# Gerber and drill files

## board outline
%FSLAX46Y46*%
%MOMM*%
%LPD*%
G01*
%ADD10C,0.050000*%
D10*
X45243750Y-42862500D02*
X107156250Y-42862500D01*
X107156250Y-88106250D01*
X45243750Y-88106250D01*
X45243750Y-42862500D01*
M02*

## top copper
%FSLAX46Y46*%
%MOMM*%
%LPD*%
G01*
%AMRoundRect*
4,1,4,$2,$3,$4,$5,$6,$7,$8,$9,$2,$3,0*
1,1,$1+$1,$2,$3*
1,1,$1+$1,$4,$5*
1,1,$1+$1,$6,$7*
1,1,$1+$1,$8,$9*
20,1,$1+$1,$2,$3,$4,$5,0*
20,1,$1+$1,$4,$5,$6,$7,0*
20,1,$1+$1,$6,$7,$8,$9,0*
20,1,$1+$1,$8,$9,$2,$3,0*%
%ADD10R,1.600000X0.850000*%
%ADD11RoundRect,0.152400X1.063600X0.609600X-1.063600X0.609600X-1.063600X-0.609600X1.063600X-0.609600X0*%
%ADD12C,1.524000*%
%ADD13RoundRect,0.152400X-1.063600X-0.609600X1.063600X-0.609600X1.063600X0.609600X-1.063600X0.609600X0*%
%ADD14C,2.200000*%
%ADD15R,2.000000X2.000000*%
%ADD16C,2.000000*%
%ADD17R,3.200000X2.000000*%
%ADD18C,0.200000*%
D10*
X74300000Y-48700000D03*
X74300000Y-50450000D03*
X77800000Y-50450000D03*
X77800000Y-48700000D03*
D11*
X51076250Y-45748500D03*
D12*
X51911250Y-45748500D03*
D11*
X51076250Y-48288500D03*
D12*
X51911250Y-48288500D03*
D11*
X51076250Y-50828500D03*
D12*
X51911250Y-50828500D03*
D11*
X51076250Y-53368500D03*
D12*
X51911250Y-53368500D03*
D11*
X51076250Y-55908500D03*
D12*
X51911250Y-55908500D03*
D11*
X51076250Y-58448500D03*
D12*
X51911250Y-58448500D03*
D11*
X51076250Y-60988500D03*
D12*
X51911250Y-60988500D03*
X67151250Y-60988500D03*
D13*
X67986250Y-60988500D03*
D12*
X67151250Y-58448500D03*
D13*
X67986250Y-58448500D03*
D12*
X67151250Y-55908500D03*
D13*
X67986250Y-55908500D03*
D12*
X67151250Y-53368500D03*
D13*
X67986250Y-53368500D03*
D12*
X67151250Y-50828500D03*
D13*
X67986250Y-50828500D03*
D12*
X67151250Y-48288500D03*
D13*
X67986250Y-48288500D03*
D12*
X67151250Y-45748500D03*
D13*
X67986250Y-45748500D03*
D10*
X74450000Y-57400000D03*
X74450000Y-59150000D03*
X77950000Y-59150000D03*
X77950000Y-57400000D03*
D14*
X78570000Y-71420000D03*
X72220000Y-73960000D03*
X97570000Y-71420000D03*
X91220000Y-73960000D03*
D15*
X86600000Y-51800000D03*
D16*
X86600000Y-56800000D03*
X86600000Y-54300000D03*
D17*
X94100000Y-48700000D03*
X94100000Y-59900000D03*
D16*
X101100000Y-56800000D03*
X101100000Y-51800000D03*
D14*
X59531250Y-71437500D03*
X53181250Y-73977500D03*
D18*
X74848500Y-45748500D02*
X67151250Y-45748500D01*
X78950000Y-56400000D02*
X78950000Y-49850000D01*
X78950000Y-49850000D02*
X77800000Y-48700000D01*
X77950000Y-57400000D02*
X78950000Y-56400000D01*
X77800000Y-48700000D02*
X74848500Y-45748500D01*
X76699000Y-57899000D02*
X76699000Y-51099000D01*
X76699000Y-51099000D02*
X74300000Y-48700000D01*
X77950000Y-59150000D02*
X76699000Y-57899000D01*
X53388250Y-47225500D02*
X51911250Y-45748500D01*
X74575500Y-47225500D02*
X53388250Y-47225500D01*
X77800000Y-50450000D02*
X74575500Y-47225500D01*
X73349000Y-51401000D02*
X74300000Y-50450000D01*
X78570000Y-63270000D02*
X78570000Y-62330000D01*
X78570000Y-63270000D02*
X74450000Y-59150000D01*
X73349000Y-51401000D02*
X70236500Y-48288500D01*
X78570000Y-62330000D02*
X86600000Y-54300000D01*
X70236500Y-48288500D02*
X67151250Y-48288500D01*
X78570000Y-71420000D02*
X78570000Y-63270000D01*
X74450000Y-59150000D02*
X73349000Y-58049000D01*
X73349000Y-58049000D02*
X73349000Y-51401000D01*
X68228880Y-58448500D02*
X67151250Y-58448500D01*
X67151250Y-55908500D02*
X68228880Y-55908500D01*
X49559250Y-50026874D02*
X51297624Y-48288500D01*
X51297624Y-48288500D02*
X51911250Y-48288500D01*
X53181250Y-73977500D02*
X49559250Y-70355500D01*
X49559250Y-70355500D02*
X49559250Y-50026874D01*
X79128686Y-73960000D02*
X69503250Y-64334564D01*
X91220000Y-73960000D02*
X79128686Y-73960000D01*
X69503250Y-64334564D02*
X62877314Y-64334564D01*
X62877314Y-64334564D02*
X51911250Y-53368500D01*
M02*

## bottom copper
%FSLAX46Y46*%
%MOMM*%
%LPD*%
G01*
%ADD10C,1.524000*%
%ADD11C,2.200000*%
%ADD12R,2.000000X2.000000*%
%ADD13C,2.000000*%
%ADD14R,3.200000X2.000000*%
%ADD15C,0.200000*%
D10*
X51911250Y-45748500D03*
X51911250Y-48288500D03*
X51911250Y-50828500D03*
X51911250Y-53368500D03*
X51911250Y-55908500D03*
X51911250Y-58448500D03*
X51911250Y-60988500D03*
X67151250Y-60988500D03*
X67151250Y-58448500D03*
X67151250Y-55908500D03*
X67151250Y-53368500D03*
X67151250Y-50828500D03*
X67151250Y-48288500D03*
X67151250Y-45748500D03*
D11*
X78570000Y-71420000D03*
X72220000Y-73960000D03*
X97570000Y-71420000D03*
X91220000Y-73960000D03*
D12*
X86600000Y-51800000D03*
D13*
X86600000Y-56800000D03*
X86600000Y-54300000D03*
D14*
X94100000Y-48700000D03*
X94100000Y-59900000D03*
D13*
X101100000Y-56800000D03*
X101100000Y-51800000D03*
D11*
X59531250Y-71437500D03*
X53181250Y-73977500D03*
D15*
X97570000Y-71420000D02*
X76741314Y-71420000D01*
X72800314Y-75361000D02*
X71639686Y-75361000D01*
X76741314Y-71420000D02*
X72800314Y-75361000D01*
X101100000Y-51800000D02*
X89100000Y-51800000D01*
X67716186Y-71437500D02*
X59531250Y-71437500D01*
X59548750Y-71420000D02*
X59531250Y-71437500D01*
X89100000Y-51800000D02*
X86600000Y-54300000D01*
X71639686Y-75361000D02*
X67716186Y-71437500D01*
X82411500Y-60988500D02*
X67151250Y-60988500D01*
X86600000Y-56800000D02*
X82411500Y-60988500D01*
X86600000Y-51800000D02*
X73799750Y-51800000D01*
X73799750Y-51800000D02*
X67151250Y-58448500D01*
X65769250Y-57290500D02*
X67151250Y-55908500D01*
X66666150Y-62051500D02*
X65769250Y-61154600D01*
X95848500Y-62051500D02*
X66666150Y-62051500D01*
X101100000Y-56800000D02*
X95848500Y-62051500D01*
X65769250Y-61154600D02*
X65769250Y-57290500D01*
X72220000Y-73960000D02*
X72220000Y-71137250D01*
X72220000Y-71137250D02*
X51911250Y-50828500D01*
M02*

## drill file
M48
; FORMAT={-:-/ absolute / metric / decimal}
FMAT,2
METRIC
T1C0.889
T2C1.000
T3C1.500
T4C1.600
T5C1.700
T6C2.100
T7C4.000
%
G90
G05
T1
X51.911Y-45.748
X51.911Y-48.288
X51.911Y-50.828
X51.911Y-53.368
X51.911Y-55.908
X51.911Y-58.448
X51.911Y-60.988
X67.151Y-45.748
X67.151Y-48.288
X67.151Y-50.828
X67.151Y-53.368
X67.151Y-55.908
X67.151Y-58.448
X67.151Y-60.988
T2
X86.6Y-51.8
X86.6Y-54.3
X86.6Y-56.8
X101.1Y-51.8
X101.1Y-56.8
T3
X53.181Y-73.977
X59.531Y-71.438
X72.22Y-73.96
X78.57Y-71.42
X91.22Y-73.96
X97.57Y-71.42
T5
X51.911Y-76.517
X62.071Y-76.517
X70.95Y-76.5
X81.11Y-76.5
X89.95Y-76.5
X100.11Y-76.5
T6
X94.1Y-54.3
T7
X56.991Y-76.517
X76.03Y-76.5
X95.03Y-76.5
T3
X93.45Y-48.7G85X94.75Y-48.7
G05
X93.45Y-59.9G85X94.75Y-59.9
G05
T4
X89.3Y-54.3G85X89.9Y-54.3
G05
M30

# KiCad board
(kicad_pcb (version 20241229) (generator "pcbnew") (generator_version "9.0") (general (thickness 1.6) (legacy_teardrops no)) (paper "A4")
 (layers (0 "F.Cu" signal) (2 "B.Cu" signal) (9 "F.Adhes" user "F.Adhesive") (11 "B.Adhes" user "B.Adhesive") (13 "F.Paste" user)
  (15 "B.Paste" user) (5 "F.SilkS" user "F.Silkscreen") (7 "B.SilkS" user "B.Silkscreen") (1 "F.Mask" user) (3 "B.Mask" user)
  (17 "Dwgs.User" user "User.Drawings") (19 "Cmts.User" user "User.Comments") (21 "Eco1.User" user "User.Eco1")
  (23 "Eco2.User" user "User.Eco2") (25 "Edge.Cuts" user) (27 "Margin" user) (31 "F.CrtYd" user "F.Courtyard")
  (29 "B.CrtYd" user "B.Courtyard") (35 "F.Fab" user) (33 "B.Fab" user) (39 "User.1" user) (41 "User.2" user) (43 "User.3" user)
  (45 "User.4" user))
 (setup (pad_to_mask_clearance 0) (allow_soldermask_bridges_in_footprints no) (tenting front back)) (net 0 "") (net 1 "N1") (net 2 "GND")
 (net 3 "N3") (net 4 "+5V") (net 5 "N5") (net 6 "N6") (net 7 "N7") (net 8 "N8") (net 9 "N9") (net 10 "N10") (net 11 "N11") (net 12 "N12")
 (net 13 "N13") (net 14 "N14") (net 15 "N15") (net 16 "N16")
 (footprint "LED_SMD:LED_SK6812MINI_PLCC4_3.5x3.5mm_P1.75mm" (layer "F.Cu") (at 76.05 49.575)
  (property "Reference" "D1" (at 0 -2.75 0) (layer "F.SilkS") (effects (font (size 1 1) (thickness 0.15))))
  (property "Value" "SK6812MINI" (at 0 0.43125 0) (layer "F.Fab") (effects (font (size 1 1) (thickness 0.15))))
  (pad "1" smd rect (at -1.75 -0.875) (size 1.6 0.85) (layers "F.Cu" "F.Mask" "F.Paste") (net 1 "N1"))
  (pad "2" smd rect (at -1.75 0.875) (size 1.6 0.85) (layers "F.Cu" "F.Mask" "F.Paste") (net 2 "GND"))
  (pad "3" smd rect (at 1.75 0.875) (size 1.6 0.85) (layers "F.Cu" "F.Mask" "F.Paste") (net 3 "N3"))
  (pad "4" smd rect (at 1.75 -0.875) (size 1.6 0.85) (layers "F.Cu" "F.Mask" "F.Paste") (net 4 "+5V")))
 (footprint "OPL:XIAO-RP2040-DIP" (layer "F.Cu") (at 59.53125 53.3685)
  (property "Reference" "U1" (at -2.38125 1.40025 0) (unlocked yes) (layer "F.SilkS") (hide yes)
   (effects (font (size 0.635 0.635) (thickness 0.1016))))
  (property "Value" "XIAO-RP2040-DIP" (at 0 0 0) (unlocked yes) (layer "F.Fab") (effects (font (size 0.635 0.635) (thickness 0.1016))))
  (pad "1" smd roundrect (at -8.455 -7.62 180) (size 2.432 1.524) (layers "F.Cu" "F.Mask") (roundrect_rratio 0.1) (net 3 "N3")
   (thermal_bridge_angle 45))
  (pad "1" thru_hole circle (at -7.62 -7.62 180) (size 1.524 1.524) (drill 0.889) (layers "*.Cu" "*.Mask") (remove_unused_layers no)
   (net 3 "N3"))
  (pad "2" smd roundrect (at -8.455 -5.08 180) (size 2.432 1.524) (layers "F.Cu" "F.Mask") (roundrect_rratio 0.1) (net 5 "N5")
   (thermal_bridge_angle 45))
  (pad "2" thru_hole circle (at -7.62 -5.08 180) (size 1.524 1.524) (drill 0.889) (layers "*.Cu" "*.Mask") (remove_unused_layers no)
   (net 5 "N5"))
  (pad "3" smd roundrect (at -8.455 -2.54 180) (size 2.432 1.524) (layers "F.Cu" "F.Mask") (roundrect_rratio 0.1) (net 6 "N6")
   (thermal_bridge_angle 45))
  (pad "3" thru_hole circle (at -7.62 -2.54 180) (size 1.524 1.524) (drill 0.889) (layers "*.Cu" "*.Mask") (remove_unused_layers no)
   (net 6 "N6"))
  (pad "4" smd roundrect (at -8.455 0 180) (size 2.432 1.524) (layers "F.Cu" "F.Mask") (roundrect_rratio 0.1) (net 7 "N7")
   (thermal_bridge_angle 45))
  (pad "4" thru_hole circle (at -7.62 0 180) (size 1.524 1.524) (drill 0.889) (layers "*.Cu" "*.Mask") (remove_unused_layers no)
   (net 7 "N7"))
  (pad "5" smd roundrect (at -8.455 2.54 180) (size 2.432 1.524) (layers "F.Cu" "F.Mask") (roundrect_rratio 0.1) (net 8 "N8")
   (thermal_bridge_angle 45))
  (pad "5" thru_hole circle (at -7.62 2.54 180) (size 1.524 1.524) (drill 0.889) (layers "*.Cu" "*.Mask") (remove_unused_layers no)
   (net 8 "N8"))
  (pad "6" smd roundrect (at -8.455 5.08 180) (size 2.432 1.524) (layers "F.Cu" "F.Mask") (roundrect_rratio 0.1) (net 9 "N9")
   (thermal_bridge_angle 45))
  (pad "6" thru_hole circle (at -7.62 5.08 180) (size 1.524 1.524) (drill 0.889) (layers "*.Cu" "*.Mask") (remove_unused_layers no)
   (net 9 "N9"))
  (pad "7" smd roundrect (at -8.455 7.62 180) (size 2.432 1.524) (layers "F.Cu" "F.Mask") (roundrect_rratio 0.1) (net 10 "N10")
   (thermal_bridge_angle 45))
  (pad "7" thru_hole circle (at -7.62 7.62 180) (size 1.524 1.524) (drill 0.889) (layers "*.Cu" "*.Mask") (remove_unused_layers no)
   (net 10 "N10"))
  (pad "8" thru_hole circle (at 7.62 7.62) (size 1.524 1.524) (drill 0.889) (layers "*.Cu" "*.Mask") (remove_unused_layers no)
   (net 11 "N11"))
  (pad "8" smd roundrect (at 8.455 7.62) (size 2.432 1.524) (layers "F.Cu" "F.Mask") (roundrect_rratio 0.1) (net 11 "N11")
   (thermal_bridge_angle 45))
  (pad "9" thru_hole circle (at 7.62 5.08) (size 1.524 1.524) (drill 0.889) (layers "*.Cu" "*.Mask") (remove_unused_layers no)
   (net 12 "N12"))
  (pad "9" smd roundrect (at 8.455 5.08) (size 2.432 1.524) (layers "F.Cu" "F.Mask") (roundrect_rratio 0.1) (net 12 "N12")
   (thermal_bridge_angle 45))
  (pad "10" thru_hole circle (at 7.62 2.54) (size 1.524 1.524) (drill 0.889) (layers "*.Cu" "*.Mask") (remove_unused_layers no)
   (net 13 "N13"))
  (pad "10" smd roundrect (at 8.455 2.54) (size 2.432 1.524) (layers "F.Cu" "F.Mask") (roundrect_rratio 0.1) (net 13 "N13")
   (thermal_bridge_angle 45))
  (pad "11" thru_hole circle (at 7.62 0) (size 1.524 1.524) (drill 0.889) (layers "*.Cu" "*.Mask") (remove_unused_layers no) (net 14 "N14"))
  (pad "11" smd roundrect (at 8.455 0) (size 2.432 1.524) (layers "F.Cu" "F.Mask") (roundrect_rratio 0.1) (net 14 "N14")
   (thermal_bridge_angle 45))
  (pad "12" thru_hole circle (at 7.62 -2.54) (size 1.524 1.524) (drill 0.889) (layers "*.Cu" "*.Mask") (remove_unused_layers no)
   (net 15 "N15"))
  (pad "12" smd roundrect (at 8.455 -2.54) (size 2.432 1.524) (layers "F.Cu" "F.Mask") (roundrect_rratio 0.1) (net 15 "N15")
   (thermal_bridge_angle 45))
  (pad "13" thru_hole circle (at 7.62 -5.08) (size 1.524 1.524) (drill 0.889) (layers "*.Cu" "*.Mask") (remove_unused_layers no)
   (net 2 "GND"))
  (pad "13" smd roundrect (at 8.455 -5.08) (size 2.432 1.524) (layers "F.Cu" "F.Mask") (roundrect_rratio 0.1) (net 2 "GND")
   (thermal_bridge_angle 45))
  (pad "14" thru_hole circle (at 7.62 -7.62) (size 1.524 1.524) (drill 0.889) (layers "*.Cu" "*.Mask") (remove_unused_layers no)
   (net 4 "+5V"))
  (pad "14" smd roundrect (at 8.455 -7.62) (size 2.432 1.524) (layers "F.Cu" "F.Mask") (roundrect_rratio 0.1) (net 4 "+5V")
   (thermal_bridge_angle 45)))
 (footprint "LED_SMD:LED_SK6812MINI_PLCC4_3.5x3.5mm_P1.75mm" (layer "F.Cu") (at 76.2 58.275)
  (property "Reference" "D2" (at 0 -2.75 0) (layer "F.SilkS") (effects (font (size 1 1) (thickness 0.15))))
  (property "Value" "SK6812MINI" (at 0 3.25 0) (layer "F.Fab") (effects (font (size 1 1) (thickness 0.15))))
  (pad "1" smd rect (at -1.75 -0.875) (size 1.6 0.85) (layers "F.Cu" "F.Mask" "F.Paste") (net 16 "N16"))
  (pad "2" smd rect (at -1.75 0.875) (size 1.6 0.85) (layers "F.Cu" "F.Mask" "F.Paste") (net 2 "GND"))
  (pad "3" smd rect (at 1.75 0.875) (size 1.6 0.85) (layers "F.Cu" "F.Mask" "F.Paste") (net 1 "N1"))
  (pad "4" smd rect (at 1.75 -0.875) (size 1.6 0.85) (layers "F.Cu" "F.Mask" "F.Paste") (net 4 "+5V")))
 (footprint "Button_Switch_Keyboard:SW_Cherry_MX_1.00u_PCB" (layer "F.Cu") (at 78.57 71.42)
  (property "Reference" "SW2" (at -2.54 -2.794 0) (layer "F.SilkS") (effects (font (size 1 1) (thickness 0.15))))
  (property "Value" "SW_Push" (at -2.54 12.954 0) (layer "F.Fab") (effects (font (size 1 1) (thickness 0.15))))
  (pad "" np_thru_hole circle (at -7.62 5.08) (size 1.7 1.7) (drill 1.7) (layers "*.Cu" "*.Mask"))
  (pad "" np_thru_hole circle (at -2.54 5.08) (size 4 4) (drill 4) (layers "*.Cu" "*.Mask"))
  (pad "" np_thru_hole circle (at 2.54 5.08) (size 1.7 1.7) (drill 1.7) (layers "*.Cu" "*.Mask"))
  (pad "1" thru_hole circle (at 0 0) (size 2.2 2.2) (drill 1.5) (layers "*.Cu" "*.Mask") (remove_unused_layers no) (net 2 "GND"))
  (pad "2" thru_hole circle (at -6.35 2.54) (size 2.2 2.2) (drill 1.5) (layers "*.Cu" "*.Mask") (remove_unused_layers no) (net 6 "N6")))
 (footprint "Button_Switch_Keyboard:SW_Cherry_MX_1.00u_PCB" (layer "F.Cu") (at 97.57 71.42)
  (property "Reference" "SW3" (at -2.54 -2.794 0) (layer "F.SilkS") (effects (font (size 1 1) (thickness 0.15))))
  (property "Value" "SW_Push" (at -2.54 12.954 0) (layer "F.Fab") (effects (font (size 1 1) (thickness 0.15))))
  (pad "" np_thru_hole circle (at -7.62 5.08) (size 1.7 1.7) (drill 1.7) (layers "*.Cu" "*.Mask"))
  (pad "" np_thru_hole circle (at -2.54 5.08) (size 4 4) (drill 4) (layers "*.Cu" "*.Mask"))
  (pad "" np_thru_hole circle (at 2.54 5.08) (size 1.7 1.7) (drill 1.7) (layers "*.Cu" "*.Mask"))
  (pad "1" thru_hole circle (at 0 0) (size 2.2 2.2) (drill 1.5) (layers "*.Cu" "*.Mask") (remove_unused_layers no) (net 2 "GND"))
  (pad "2" thru_hole circle (at -6.35 2.54) (size 2.2 2.2) (drill 1.5) (layers "*.Cu" "*.Mask") (remove_unused_layers no) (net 7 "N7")))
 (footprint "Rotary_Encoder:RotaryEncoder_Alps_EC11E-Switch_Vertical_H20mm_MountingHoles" (layer "F.Cu") (at 86.6 51.8)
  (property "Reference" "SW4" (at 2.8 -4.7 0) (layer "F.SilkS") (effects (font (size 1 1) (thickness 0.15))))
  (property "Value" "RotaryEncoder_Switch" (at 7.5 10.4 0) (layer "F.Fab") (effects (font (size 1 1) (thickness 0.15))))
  (pad "" np_thru_hole oval (at 3 2.5) (size 2.2 1.6) (drill oval 2.2 1.6) (layers "*.Mask"))
  (pad "" np_thru_hole circle (at 7.5 2.5) (size 2.1 2.1) (drill 2.1) (layers "*.Mask"))
  (pad "A" thru_hole rect (at 0 0) (size 2 2) (drill 1) (layers "*.Cu" "*.Mask") (remove_unused_layers no) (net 12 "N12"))
  (pad "B" thru_hole circle (at 0 5) (size 2 2) (drill 1) (layers "*.Cu" "*.Mask") (remove_unused_layers no) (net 11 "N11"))
  (pad "C" thru_hole circle (at 0 2.5) (size 2 2) (drill 1) (layers "*.Cu" "*.Mask") (remove_unused_layers no) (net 2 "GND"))
  (pad "MP" thru_hole rect (at 7.5 -3.1) (size 3.2 2) (drill oval 2.8 1.5) (layers "*.Cu" "*.Mask") (remove_unused_layers no))
  (pad "MP" thru_hole rect (at 7.5 8.1) (size 3.2 2) (drill oval 2.8 1.5) (layers "*.Cu" "*.Mask") (remove_unused_layers no))
  (pad "S1" thru_hole circle (at 14.5 5) (size 2 2) (drill 1) (layers "*.Cu" "*.Mask") (remove_unused_layers no) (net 13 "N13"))
  (pad "S2" thru_hole circle (at 14.5 0) (size 2 2) (drill 1) (layers "*.Cu" "*.Mask") (remove_unused_layers no) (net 2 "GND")))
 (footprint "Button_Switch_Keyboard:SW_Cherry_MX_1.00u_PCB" (layer "F.Cu") (at 59.53125 71.4375)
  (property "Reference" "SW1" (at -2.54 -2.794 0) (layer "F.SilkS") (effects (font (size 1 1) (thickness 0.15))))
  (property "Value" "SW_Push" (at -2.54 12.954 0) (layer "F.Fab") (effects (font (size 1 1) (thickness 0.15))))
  (pad "" np_thru_hole circle (at -7.62 5.08) (size 1.7 1.7) (drill 1.7) (layers "*.Cu" "*.Mask"))
  (pad "" np_thru_hole circle (at -2.54 5.08) (size 4 4) (drill 4) (layers "*.Cu" "*.Mask"))
  (pad "" np_thru_hole circle (at 2.54 5.08) (size 1.7 1.7) (drill 1.7) (layers "*.Cu" "*.Mask"))
  (pad "1" thru_hole circle (at 0 0) (size 2.2 2.2) (drill 1.5) (layers "*.Cu" "*.Mask") (remove_unused_layers no) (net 2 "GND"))
  (pad "2" thru_hole circle (at -6.35 2.54) (size 2.2 2.2) (drill 1.5) (layers "*.Cu" "*.Mask") (remove_unused_layers no) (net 5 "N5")))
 (gr_rect (start 45.24375 42.8625) (end 107.15625 88.10625) (stroke (width 0.05) (type default)) (fill no) (layer "Edge.Cuts"))
 (segment (start 74.8485 45.7485) (end 67.15125 45.7485) (width 0.2) (layer "F.Cu") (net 4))
 (segment (start 78.95 56.4) (end 78.95 49.85) (width 0.2) (layer "F.Cu") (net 4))
 (segment (start 78.95 49.85) (end 77.8 48.7) (width 0.2) (layer "F.Cu") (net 4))
 (segment (start 77.95 57.4) (end 78.95 56.4) (width 0.2) (layer "F.Cu") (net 4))
 (segment (start 77.8 48.7) (end 74.8485 45.7485) (width 0.2) (layer "F.Cu") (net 4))
 (segment (start 76.699 57.899) (end 76.699 51.099) (width 0.2) (layer "F.Cu") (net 1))
 (segment (start 76.699 51.099) (end 74.3 48.7) (width 0.2) (layer "F.Cu") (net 1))
 (segment (start 77.95 59.15) (end 76.699 57.899) (width 0.2) (layer "F.Cu") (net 1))
 (segment (start 53.38825 47.2255) (end 51.91125 45.7485) (width 0.2) (layer "F.Cu") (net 3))
 (segment (start 74.5755 47.2255) (end 53.38825 47.2255) (width 0.2) (layer "F.Cu") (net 3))
 (segment (start 77.8 50.45) (end 74.5755 47.2255) (width 0.2) (layer "F.Cu") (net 3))
 (segment (start 73.349 51.401) (end 74.3 50.45) (width 0.2) (layer "F.Cu") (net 2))
 (segment (start 78.57 63.27) (end 78.57 62.33) (width 0.2) (layer "F.Cu") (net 2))
 (segment (start 78.57 63.27) (end 74.45 59.15) (width 0.2) (layer "F.Cu") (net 2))
 (segment (start 73.349 51.401) (end 70.2365 48.2885) (width 0.2) (layer "F.Cu") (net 2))
 (segment (start 78.57 62.33) (end 86.6 54.3) (width 0.2) (layer "F.Cu") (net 2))
 (segment (start 70.2365 48.2885) (end 67.15125 48.2885) (width 0.2) (layer "F.Cu") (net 2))
 (segment (start 78.57 71.42) (end 78.57 63.27) (width 0.2) (layer "F.Cu") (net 2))
 (segment (start 74.45 59.15) (end 73.349 58.049) (width 0.2) (layer "F.Cu") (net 2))
 (segment (start 73.349 58.049) (end 73.349 51.401) (width 0.2) (layer "F.Cu") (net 2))
 (segment (start 97.57 71.42) (end 76.741314 71.42) (width 0.2) (layer "B.Cu") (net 2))
 (segment (start 72.800314 75.361) (end 71.639686 75.361) (width 0.2) (layer "B.Cu") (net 2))
 (segment (start 76.741314 71.42) (end 72.800314 75.361) (width 0.2) (layer "B.Cu") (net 2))
 (segment (start 101.1 51.8) (end 89.1 51.8) (width 0.2) (layer "B.Cu") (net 2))
 (segment (start 67.716186 71.4375) (end 59.53125 71.4375) (width 0.2) (layer "B.Cu") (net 2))
 (segment (start 59.54875 71.42) (end 59.53125 71.4375) (width 0.2) (layer "B.Cu") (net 2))
 (segment (start 89.1 51.8) (end 86.6 54.3) (width 0.2) (layer "B.Cu") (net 2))
 (segment (start 71.639686 75.361) (end 67.716186 71.4375) (width 0.2) (layer "B.Cu") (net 2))
 (segment (start 82.4115 60.9885) (end 67.15125 60.9885) (width 0.2) (layer "B.Cu") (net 11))
 (segment (start 86.6 56.8) (end 82.4115 60.9885) (width 0.2) (layer "B.Cu") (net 11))
 (segment (start 68.22888 58.4485) (end 67.15125 58.4485) (width 0.2) (layer "F.Cu") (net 12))
 (segment (start 86.6 51.8) (end 73.79975 51.8) (width 0.2) (layer "B.Cu") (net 12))
 (segment (start 73.79975 51.8) (end 67.15125 58.4485) (width 0.2) (layer "B.Cu") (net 12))
 (segment (start 67.15125 55.9085) (end 68.22888 55.9085) (width 0.2) (layer "F.Cu") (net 13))
 (segment (start 65.76925 57.2905) (end 67.15125 55.9085) (width 0.2) (layer "B.Cu") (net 13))
 (segment (start 66.66615 62.0515) (end 65.76925 61.1546) (width 0.2) (layer "B.Cu") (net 13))
 (segment (start 95.8485 62.0515) (end 66.66615 62.0515) (width 0.2) (layer "B.Cu") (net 13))
 (segment (start 101.1 56.8) (end 95.8485 62.0515) (width 0.2) (layer "B.Cu") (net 13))
 (segment (start 65.76925 61.1546) (end 65.76925 57.2905) (width 0.2) (layer "B.Cu") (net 13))
 (segment (start 49.55925 50.026874) (end 51.297624 48.2885) (width 0.2) (layer "F.Cu") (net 5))
 (segment (start 51.297624 48.2885) (end 51.91125 48.2885) (width 0.2) (layer "F.Cu") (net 5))
 (segment (start 53.18125 73.9775) (end 49.55925 70.3555) (width 0.2) (layer "F.Cu") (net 5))
 (segment (start 49.55925 70.3555) (end 49.55925 50.026874) (width 0.2) (layer "F.Cu") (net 5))
 (segment (start 72.22 73.96) (end 72.22 71.13725) (width 0.2) (layer "B.Cu") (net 6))
 (segment (start 72.22 71.13725) (end 51.91125 50.8285) (width 0.2) (layer "B.Cu") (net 6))
 (segment (start 79.128686 73.96) (end 69.50325 64.334564) (width 0.2) (layer "F.Cu") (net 7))
 (segment (start 91.22 73.96) (end 79.128686 73.96) (width 0.2) (layer "F.Cu") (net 7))
 (segment (start 69.50325 64.334564) (end 62.877314 64.334564) (width 0.2) (layer "F.Cu") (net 7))
 (segment (start 62.877314 64.334564) (end 51.91125 53.3685) (width 0.2) (layer "F.Cu") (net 7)))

